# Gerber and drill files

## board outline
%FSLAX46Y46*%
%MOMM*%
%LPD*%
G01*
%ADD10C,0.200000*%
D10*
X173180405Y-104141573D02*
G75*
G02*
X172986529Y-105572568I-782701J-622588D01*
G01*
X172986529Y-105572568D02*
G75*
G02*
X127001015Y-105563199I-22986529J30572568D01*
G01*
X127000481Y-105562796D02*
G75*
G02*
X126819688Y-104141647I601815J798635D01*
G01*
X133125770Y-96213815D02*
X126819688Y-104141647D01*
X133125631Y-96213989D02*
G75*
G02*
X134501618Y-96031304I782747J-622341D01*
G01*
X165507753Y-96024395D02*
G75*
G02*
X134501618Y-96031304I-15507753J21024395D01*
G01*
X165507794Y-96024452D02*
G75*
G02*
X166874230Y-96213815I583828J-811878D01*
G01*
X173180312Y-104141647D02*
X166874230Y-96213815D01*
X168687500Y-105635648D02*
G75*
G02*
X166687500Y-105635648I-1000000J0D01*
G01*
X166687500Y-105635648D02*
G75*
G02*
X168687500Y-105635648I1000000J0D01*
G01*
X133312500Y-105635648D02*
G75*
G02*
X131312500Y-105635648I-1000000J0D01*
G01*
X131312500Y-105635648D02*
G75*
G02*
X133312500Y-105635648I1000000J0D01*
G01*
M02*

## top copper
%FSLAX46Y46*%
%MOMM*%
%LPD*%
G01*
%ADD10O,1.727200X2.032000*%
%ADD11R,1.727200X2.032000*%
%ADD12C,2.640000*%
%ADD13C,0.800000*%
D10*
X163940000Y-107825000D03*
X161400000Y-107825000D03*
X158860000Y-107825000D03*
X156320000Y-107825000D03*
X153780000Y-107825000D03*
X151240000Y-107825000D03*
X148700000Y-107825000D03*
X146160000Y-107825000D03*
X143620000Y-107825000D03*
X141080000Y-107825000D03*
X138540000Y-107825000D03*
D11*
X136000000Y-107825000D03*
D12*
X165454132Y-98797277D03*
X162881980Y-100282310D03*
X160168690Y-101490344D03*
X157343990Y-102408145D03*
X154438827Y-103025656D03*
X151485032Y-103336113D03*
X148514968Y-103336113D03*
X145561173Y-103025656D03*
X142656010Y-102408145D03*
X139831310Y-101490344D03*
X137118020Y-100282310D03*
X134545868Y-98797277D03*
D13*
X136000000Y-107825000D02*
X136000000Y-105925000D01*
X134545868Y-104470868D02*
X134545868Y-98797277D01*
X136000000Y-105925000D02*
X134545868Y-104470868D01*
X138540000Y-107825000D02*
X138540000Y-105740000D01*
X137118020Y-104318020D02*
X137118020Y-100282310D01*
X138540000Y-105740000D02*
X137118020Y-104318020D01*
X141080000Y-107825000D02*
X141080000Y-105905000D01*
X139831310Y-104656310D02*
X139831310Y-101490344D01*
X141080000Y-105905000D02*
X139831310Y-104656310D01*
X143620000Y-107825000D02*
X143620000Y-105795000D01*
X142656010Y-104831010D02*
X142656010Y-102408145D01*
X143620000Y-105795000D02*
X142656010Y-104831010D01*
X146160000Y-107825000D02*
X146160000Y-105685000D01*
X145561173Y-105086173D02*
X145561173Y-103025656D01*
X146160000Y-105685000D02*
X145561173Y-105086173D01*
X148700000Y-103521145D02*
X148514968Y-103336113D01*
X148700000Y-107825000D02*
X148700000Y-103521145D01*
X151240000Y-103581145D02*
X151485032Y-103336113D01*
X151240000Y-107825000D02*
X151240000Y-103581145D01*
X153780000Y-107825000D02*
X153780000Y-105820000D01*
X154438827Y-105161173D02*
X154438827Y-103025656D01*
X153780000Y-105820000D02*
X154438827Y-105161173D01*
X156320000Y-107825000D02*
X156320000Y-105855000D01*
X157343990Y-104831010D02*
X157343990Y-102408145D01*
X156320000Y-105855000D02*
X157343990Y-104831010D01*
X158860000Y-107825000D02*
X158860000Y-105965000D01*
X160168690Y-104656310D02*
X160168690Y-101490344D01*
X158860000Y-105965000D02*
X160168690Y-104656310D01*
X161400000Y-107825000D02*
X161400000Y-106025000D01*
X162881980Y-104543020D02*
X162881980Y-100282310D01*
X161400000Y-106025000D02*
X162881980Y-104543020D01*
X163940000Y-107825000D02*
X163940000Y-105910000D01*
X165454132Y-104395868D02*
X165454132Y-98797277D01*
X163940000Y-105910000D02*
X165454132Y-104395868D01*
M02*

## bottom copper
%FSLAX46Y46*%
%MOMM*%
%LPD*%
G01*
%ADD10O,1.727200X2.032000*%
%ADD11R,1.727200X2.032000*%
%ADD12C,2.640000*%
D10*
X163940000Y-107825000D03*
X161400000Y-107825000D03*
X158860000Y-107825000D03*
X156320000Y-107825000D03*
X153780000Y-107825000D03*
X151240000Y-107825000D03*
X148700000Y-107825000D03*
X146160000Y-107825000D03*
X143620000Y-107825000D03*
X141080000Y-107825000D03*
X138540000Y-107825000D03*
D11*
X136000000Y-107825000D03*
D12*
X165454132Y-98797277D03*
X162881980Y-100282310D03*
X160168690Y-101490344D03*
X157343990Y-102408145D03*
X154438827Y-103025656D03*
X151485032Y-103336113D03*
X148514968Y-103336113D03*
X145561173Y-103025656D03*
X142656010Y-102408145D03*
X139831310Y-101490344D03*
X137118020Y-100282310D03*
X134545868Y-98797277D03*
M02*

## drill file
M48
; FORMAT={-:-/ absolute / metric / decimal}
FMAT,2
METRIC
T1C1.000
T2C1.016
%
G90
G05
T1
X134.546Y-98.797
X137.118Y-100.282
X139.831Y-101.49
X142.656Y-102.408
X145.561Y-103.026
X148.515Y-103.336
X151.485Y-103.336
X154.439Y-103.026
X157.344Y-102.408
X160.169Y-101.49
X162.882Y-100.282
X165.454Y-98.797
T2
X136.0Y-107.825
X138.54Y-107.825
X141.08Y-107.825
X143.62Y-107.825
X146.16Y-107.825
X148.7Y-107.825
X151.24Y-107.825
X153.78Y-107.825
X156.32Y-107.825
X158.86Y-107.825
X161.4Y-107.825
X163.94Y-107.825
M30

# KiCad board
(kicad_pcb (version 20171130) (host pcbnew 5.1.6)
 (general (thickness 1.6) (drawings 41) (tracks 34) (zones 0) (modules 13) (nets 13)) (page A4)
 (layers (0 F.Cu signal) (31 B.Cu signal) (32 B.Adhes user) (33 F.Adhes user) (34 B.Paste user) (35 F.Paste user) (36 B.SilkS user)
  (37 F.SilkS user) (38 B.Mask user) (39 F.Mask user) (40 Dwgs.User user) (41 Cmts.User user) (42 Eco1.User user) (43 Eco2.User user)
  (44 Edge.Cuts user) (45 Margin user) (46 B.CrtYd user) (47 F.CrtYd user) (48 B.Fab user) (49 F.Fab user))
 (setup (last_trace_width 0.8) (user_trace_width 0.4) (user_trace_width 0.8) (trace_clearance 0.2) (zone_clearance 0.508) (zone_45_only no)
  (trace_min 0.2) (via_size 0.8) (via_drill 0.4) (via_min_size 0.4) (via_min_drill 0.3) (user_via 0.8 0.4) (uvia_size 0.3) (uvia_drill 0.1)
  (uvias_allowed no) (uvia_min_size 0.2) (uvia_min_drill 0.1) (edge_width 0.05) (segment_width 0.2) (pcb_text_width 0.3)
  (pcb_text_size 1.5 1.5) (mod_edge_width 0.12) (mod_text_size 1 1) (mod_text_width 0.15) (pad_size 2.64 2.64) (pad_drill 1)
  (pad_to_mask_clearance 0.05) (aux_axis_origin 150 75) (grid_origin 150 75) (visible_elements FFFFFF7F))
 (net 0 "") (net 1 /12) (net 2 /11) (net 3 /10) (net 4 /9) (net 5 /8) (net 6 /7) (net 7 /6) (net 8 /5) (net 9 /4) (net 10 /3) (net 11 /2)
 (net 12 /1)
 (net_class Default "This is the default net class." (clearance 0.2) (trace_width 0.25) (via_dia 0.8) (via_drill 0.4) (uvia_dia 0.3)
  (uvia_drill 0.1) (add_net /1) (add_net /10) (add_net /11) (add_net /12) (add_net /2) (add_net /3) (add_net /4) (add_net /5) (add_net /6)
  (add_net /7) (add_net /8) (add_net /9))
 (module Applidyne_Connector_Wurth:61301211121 (layer B.Cu) (at 136 107.825 270)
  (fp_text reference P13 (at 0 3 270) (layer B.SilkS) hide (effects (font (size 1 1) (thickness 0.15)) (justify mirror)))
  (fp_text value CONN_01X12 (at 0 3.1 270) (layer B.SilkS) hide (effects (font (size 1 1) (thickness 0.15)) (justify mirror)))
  (pad 12 thru_hole oval (at 0 -27.94 270) (size 2.032 1.7272) (drill 1.016) (layers *.Cu *.Mask B.SilkS) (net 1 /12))
  (pad 11 thru_hole oval (at 0 -25.4 270) (size 2.032 1.7272) (drill 1.016) (layers *.Cu *.Mask B.SilkS) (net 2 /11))
  (pad 10 thru_hole oval (at 0 -22.86 270) (size 2.032 1.7272) (drill 1.016) (layers *.Cu *.Mask B.SilkS) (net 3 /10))
  (pad 9 thru_hole oval (at 0 -20.32 270) (size 2.032 1.7272) (drill 1.016) (layers *.Cu *.Mask B.SilkS) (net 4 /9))
  (pad 8 thru_hole oval (at 0 -17.78 270) (size 2.032 1.7272) (drill 1.016) (layers *.Cu *.Mask B.SilkS) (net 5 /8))
  (pad 7 thru_hole oval (at 0 -15.24 270) (size 2.032 1.7272) (drill 1.016) (layers *.Cu *.Mask B.SilkS) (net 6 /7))
  (pad 6 thru_hole oval (at 0 -12.7 270) (size 2.032 1.7272) (drill 1.016) (layers *.Cu *.Mask B.SilkS) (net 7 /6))
  (pad 5 thru_hole oval (at 0 -10.16 270) (size 2.032 1.7272) (drill 1.016) (layers *.Cu *.Mask B.SilkS) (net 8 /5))
  (pad 4 thru_hole oval (at 0 -7.62 270) (size 2.032 1.7272) (drill 1.016) (layers *.Cu *.Mask B.SilkS) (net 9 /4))
  (pad 3 thru_hole oval (at 0 -5.08 270) (size 2.032 1.7272) (drill 1.016) (layers *.Cu *.Mask B.SilkS) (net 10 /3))
  (pad 2 thru_hole oval (at 0 -2.54 270) (size 2.032 1.7272) (drill 1.016) (layers *.Cu *.Mask B.SilkS) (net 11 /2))
  (pad 1 thru_hole rect (at 0 0 270) (size 2.032 1.7272) (drill 1.016) (layers *.Cu *.Mask B.SilkS) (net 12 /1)))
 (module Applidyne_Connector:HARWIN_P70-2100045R (layer F.Cu) (at 165.454132 98.797277)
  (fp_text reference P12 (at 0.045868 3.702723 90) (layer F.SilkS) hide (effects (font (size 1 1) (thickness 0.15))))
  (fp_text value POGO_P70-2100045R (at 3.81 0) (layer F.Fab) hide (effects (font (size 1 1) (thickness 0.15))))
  (pad 1 thru_hole circle (at 0 0) (size 2.64 2.64) (drill 1) (layers *.Cu *.Mask) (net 1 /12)))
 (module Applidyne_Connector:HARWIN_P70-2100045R (layer F.Cu) (at 162.88198 100.28231)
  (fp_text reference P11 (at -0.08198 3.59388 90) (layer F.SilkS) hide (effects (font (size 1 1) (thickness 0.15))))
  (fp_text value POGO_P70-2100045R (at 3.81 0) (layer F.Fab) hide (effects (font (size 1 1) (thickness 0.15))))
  (pad 1 thru_hole circle (at 0 0) (size 2.64 2.64) (drill 1) (layers *.Cu *.Mask) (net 2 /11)))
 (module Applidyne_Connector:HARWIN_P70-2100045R (layer F.Cu) (at 160.16869 101.490344)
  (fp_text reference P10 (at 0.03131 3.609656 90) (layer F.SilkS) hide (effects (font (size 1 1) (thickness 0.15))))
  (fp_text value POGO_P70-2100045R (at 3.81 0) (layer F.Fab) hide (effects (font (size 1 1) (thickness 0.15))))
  (pad 1 thru_hole circle (at 0 0) (size 2.64 2.64) (drill 1) (layers *.Cu *.Mask) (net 3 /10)))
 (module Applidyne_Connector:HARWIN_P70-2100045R (layer F.Cu) (at 157.34399 102.408145)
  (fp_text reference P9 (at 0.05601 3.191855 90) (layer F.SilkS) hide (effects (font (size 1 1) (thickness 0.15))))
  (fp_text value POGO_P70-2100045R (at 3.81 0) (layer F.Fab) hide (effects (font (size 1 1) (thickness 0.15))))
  (pad 1 thru_hole circle (at 0 0) (size 2.64 2.64) (drill 1) (layers *.Cu *.Mask) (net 4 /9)))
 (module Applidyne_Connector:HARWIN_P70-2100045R (layer F.Cu) (at 154.438827 103.025656)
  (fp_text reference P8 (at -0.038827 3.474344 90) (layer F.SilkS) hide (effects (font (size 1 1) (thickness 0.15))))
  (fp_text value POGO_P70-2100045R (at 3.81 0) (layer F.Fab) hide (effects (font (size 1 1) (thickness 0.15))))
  (pad 1 thru_hole circle (at 0 0) (size 2.64 2.64) (drill 1) (layers *.Cu *.Mask) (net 5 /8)))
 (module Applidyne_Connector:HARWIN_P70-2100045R (layer F.Cu) (at 151.485032 103.336113)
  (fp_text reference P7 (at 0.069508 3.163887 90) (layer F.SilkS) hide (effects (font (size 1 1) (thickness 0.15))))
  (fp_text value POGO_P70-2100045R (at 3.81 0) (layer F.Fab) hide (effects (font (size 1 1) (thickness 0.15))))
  (pad 1 thru_hole circle (at 0 0) (size 2.64 2.64) (drill 1) (layers *.Cu *.Mask) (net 6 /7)))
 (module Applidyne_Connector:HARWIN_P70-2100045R (layer F.Cu) (at 148.514968 103.336113)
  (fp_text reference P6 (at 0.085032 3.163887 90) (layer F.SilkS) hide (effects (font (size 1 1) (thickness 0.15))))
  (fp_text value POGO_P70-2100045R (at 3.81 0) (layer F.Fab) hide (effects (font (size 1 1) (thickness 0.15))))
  (pad 1 thru_hole circle (at 0 0) (size 2.64 2.64) (drill 1) (layers *.Cu *.Mask) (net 7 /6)))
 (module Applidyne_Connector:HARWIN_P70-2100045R (layer F.Cu) (at 145.561173 103.025656)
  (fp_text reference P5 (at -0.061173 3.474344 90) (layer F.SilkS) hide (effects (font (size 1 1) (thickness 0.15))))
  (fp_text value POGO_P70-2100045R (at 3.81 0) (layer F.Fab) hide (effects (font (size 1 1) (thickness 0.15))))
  (pad 1 thru_hole circle (at 0 0) (size 2.64 2.64) (drill 1) (layers *.Cu *.Mask) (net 8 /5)))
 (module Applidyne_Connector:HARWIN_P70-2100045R (layer F.Cu) (at 142.65601 102.408145)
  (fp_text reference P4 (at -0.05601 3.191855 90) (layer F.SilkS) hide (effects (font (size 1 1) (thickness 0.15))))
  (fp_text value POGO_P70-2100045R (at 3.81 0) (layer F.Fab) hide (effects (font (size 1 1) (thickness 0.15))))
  (pad 1 thru_hole circle (at 0 0) (size 2.64 2.64) (drill 1) (layers *.Cu *.Mask) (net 9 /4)))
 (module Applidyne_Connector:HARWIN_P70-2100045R (layer F.Cu) (at 139.83131 101.490344)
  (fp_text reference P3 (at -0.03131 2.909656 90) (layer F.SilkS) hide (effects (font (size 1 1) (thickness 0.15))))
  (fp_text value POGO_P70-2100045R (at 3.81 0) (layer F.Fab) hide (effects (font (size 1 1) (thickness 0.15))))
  (pad 1 thru_hole circle (at 0 0) (size 2.64 2.64) (drill 1) (layers *.Cu *.Mask) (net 10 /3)))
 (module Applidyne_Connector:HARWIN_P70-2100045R (layer F.Cu) (at 137.11802 100.28231)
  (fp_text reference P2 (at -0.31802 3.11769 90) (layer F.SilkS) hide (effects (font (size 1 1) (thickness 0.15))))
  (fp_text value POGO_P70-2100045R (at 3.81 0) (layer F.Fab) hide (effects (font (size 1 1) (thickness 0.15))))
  (pad 1 thru_hole circle (at 0 0) (size 2.64 2.64) (drill 1) (layers *.Cu *.Mask) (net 11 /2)))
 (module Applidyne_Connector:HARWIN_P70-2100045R (layer F.Cu) (at 134.545868 98.797277)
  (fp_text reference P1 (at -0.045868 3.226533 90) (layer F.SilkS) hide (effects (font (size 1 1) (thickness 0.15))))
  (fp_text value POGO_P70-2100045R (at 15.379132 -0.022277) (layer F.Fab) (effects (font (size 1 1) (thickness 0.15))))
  (pad 1 thru_hole circle (at 0 0) (size 2.64 2.64) (drill 1) (layers *.Cu *.Mask) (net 12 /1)))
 (gr_arc (start 172.397704 104.764161) (end 172.986529 105.572568) (angle -92.43124742) (layer Edge.Cuts) (width 0.2))
 (gr_arc (start 150 75) (end 127.001015 105.563199) (angle -73.9) (layer Edge.Cuts) (width 0.2))
 (gr_arc (start 127.602296 104.764161) (end 126.819688 104.141647) (angle -91.49996052) (layer Edge.Cuts) (width 0.2))
 (gr_line (start 133.12577 96.213815) (end 126.819688 104.141647) (layer Edge.Cuts) (width 0.2))
 (gr_arc (start 133.908378 96.83633) (end 134.501618 96.031304) (angle -87.89999341) (layer Edge.Cuts) (width 0.2))
 (gr_arc (start 150 75) (end 134.501618 96.031304) (angle -72.8) (layer Edge.Cuts) (width 0.2))
 (gr_arc (start 166.091622 96.83633) (end 166.87423 96.213815) (angle -87.22019376) (layer Edge.Cuts) (width 0.2))
 (gr_line (start 173.180312 104.141647) (end 166.87423 96.213815) (layer Edge.Cuts) (width 0.2))
 (gr_circle (center 167.6875 105.635648) (end 168.6875 105.635648) (layer Edge.Cuts) (width 0.2))
 (gr_circle (center 132.3125 105.635648) (end 133.3125 105.635648) (layer Edge.Cuts) (width 0.2))
 (segment (start 136 107.825) (end 136 105.925) (width 0.8) (layer F.Cu) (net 12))
 (segment (start 134.545868 104.470868) (end 134.545868 98.797277) (width 0.8) (layer F.Cu) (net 12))
 (segment (start 136 105.925) (end 134.545868 104.470868) (width 0.8) (layer F.Cu) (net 12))
 (segment (start 138.54 107.825) (end 138.54 105.74) (width 0.8) (layer F.Cu) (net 11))
 (segment (start 137.11802 104.31802) (end 137.11802 100.28231) (width 0.8) (layer F.Cu) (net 11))
 (segment (start 138.54 105.74) (end 137.11802 104.31802) (width 0.8) (layer F.Cu) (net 11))
 (segment (start 141.08 107.825) (end 141.08 105.905) (width 0.8) (layer F.Cu) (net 10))
 (segment (start 139.83131 104.65631) (end 139.83131 101.490344) (width 0.8) (layer F.Cu) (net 10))
 (segment (start 141.08 105.905) (end 139.83131 104.65631) (width 0.8) (layer F.Cu) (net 10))
 (segment (start 143.62 107.825) (end 143.62 105.795) (width 0.8) (layer F.Cu) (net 9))
 (segment (start 142.65601 104.83101) (end 142.65601 102.408145) (width 0.8) (layer F.Cu) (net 9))
 (segment (start 143.62 105.795) (end 142.65601 104.83101) (width 0.8) (layer F.Cu) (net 9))
 (segment (start 146.16 107.825) (end 146.16 105.685) (width 0.8) (layer F.Cu) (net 8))
 (segment (start 145.561173 105.086173) (end 145.561173 103.025656) (width 0.8) (layer F.Cu) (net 8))
 (segment (start 146.16 105.685) (end 145.561173 105.086173) (width 0.8) (layer F.Cu) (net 8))
 (segment (start 148.7 103.521145) (end 148.514968 103.336113) (width 0.8) (layer F.Cu) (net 7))
 (segment (start 148.7 107.825) (end 148.7 103.521145) (width 0.8) (layer F.Cu) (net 7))
 (segment (start 151.24 103.581145) (end 151.485032 103.336113) (width 0.8) (layer F.Cu) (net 6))
 (segment (start 151.24 107.825) (end 151.24 103.581145) (width 0.8) (layer F.Cu) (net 6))
 (segment (start 153.78 107.825) (end 153.78 105.82) (width 0.8) (layer F.Cu) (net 5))
 (segment (start 154.438827 105.161173) (end 154.438827 103.025656) (width 0.8) (layer F.Cu) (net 5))
 (segment (start 153.78 105.82) (end 154.438827 105.161173) (width 0.8) (layer F.Cu) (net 5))
 (segment (start 156.32 107.825) (end 156.32 105.855) (width 0.8) (layer F.Cu) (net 4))
 (segment (start 157.34399 104.83101) (end 157.34399 102.408145) (width 0.8) (layer F.Cu) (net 4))
 (segment (start 156.32 105.855) (end 157.34399 104.83101) (width 0.8) (layer F.Cu) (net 4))
 (segment (start 158.86 107.825) (end 158.86 105.965) (width 0.8) (layer F.Cu) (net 3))
 (segment (start 160.16869 104.65631) (end 160.16869 101.490344) (width 0.8) (layer F.Cu) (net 3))
 (segment (start 158.86 105.965) (end 160.16869 104.65631) (width 0.8) (layer F.Cu) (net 3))
 (segment (start 161.4 107.825) (end 161.4 106.025) (width 0.8) (layer F.Cu) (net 2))
 (segment (start 162.88198 104.54302) (end 162.88198 100.28231) (width 0.8) (layer F.Cu) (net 2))
 (segment (start 161.4 106.025) (end 162.88198 104.54302) (width 0.8) (layer F.Cu) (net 2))
 (segment (start 163.94 107.825) (end 163.94 105.91) (width 0.8) (layer F.Cu) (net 1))
 (segment (start 165.454132 104.395868) (end 165.454132 98.797277) (width 0.8) (layer F.Cu) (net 1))
 (segment (start 163.94 105.91) (end 165.454132 104.395868) (width 0.8) (layer F.Cu) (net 1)))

